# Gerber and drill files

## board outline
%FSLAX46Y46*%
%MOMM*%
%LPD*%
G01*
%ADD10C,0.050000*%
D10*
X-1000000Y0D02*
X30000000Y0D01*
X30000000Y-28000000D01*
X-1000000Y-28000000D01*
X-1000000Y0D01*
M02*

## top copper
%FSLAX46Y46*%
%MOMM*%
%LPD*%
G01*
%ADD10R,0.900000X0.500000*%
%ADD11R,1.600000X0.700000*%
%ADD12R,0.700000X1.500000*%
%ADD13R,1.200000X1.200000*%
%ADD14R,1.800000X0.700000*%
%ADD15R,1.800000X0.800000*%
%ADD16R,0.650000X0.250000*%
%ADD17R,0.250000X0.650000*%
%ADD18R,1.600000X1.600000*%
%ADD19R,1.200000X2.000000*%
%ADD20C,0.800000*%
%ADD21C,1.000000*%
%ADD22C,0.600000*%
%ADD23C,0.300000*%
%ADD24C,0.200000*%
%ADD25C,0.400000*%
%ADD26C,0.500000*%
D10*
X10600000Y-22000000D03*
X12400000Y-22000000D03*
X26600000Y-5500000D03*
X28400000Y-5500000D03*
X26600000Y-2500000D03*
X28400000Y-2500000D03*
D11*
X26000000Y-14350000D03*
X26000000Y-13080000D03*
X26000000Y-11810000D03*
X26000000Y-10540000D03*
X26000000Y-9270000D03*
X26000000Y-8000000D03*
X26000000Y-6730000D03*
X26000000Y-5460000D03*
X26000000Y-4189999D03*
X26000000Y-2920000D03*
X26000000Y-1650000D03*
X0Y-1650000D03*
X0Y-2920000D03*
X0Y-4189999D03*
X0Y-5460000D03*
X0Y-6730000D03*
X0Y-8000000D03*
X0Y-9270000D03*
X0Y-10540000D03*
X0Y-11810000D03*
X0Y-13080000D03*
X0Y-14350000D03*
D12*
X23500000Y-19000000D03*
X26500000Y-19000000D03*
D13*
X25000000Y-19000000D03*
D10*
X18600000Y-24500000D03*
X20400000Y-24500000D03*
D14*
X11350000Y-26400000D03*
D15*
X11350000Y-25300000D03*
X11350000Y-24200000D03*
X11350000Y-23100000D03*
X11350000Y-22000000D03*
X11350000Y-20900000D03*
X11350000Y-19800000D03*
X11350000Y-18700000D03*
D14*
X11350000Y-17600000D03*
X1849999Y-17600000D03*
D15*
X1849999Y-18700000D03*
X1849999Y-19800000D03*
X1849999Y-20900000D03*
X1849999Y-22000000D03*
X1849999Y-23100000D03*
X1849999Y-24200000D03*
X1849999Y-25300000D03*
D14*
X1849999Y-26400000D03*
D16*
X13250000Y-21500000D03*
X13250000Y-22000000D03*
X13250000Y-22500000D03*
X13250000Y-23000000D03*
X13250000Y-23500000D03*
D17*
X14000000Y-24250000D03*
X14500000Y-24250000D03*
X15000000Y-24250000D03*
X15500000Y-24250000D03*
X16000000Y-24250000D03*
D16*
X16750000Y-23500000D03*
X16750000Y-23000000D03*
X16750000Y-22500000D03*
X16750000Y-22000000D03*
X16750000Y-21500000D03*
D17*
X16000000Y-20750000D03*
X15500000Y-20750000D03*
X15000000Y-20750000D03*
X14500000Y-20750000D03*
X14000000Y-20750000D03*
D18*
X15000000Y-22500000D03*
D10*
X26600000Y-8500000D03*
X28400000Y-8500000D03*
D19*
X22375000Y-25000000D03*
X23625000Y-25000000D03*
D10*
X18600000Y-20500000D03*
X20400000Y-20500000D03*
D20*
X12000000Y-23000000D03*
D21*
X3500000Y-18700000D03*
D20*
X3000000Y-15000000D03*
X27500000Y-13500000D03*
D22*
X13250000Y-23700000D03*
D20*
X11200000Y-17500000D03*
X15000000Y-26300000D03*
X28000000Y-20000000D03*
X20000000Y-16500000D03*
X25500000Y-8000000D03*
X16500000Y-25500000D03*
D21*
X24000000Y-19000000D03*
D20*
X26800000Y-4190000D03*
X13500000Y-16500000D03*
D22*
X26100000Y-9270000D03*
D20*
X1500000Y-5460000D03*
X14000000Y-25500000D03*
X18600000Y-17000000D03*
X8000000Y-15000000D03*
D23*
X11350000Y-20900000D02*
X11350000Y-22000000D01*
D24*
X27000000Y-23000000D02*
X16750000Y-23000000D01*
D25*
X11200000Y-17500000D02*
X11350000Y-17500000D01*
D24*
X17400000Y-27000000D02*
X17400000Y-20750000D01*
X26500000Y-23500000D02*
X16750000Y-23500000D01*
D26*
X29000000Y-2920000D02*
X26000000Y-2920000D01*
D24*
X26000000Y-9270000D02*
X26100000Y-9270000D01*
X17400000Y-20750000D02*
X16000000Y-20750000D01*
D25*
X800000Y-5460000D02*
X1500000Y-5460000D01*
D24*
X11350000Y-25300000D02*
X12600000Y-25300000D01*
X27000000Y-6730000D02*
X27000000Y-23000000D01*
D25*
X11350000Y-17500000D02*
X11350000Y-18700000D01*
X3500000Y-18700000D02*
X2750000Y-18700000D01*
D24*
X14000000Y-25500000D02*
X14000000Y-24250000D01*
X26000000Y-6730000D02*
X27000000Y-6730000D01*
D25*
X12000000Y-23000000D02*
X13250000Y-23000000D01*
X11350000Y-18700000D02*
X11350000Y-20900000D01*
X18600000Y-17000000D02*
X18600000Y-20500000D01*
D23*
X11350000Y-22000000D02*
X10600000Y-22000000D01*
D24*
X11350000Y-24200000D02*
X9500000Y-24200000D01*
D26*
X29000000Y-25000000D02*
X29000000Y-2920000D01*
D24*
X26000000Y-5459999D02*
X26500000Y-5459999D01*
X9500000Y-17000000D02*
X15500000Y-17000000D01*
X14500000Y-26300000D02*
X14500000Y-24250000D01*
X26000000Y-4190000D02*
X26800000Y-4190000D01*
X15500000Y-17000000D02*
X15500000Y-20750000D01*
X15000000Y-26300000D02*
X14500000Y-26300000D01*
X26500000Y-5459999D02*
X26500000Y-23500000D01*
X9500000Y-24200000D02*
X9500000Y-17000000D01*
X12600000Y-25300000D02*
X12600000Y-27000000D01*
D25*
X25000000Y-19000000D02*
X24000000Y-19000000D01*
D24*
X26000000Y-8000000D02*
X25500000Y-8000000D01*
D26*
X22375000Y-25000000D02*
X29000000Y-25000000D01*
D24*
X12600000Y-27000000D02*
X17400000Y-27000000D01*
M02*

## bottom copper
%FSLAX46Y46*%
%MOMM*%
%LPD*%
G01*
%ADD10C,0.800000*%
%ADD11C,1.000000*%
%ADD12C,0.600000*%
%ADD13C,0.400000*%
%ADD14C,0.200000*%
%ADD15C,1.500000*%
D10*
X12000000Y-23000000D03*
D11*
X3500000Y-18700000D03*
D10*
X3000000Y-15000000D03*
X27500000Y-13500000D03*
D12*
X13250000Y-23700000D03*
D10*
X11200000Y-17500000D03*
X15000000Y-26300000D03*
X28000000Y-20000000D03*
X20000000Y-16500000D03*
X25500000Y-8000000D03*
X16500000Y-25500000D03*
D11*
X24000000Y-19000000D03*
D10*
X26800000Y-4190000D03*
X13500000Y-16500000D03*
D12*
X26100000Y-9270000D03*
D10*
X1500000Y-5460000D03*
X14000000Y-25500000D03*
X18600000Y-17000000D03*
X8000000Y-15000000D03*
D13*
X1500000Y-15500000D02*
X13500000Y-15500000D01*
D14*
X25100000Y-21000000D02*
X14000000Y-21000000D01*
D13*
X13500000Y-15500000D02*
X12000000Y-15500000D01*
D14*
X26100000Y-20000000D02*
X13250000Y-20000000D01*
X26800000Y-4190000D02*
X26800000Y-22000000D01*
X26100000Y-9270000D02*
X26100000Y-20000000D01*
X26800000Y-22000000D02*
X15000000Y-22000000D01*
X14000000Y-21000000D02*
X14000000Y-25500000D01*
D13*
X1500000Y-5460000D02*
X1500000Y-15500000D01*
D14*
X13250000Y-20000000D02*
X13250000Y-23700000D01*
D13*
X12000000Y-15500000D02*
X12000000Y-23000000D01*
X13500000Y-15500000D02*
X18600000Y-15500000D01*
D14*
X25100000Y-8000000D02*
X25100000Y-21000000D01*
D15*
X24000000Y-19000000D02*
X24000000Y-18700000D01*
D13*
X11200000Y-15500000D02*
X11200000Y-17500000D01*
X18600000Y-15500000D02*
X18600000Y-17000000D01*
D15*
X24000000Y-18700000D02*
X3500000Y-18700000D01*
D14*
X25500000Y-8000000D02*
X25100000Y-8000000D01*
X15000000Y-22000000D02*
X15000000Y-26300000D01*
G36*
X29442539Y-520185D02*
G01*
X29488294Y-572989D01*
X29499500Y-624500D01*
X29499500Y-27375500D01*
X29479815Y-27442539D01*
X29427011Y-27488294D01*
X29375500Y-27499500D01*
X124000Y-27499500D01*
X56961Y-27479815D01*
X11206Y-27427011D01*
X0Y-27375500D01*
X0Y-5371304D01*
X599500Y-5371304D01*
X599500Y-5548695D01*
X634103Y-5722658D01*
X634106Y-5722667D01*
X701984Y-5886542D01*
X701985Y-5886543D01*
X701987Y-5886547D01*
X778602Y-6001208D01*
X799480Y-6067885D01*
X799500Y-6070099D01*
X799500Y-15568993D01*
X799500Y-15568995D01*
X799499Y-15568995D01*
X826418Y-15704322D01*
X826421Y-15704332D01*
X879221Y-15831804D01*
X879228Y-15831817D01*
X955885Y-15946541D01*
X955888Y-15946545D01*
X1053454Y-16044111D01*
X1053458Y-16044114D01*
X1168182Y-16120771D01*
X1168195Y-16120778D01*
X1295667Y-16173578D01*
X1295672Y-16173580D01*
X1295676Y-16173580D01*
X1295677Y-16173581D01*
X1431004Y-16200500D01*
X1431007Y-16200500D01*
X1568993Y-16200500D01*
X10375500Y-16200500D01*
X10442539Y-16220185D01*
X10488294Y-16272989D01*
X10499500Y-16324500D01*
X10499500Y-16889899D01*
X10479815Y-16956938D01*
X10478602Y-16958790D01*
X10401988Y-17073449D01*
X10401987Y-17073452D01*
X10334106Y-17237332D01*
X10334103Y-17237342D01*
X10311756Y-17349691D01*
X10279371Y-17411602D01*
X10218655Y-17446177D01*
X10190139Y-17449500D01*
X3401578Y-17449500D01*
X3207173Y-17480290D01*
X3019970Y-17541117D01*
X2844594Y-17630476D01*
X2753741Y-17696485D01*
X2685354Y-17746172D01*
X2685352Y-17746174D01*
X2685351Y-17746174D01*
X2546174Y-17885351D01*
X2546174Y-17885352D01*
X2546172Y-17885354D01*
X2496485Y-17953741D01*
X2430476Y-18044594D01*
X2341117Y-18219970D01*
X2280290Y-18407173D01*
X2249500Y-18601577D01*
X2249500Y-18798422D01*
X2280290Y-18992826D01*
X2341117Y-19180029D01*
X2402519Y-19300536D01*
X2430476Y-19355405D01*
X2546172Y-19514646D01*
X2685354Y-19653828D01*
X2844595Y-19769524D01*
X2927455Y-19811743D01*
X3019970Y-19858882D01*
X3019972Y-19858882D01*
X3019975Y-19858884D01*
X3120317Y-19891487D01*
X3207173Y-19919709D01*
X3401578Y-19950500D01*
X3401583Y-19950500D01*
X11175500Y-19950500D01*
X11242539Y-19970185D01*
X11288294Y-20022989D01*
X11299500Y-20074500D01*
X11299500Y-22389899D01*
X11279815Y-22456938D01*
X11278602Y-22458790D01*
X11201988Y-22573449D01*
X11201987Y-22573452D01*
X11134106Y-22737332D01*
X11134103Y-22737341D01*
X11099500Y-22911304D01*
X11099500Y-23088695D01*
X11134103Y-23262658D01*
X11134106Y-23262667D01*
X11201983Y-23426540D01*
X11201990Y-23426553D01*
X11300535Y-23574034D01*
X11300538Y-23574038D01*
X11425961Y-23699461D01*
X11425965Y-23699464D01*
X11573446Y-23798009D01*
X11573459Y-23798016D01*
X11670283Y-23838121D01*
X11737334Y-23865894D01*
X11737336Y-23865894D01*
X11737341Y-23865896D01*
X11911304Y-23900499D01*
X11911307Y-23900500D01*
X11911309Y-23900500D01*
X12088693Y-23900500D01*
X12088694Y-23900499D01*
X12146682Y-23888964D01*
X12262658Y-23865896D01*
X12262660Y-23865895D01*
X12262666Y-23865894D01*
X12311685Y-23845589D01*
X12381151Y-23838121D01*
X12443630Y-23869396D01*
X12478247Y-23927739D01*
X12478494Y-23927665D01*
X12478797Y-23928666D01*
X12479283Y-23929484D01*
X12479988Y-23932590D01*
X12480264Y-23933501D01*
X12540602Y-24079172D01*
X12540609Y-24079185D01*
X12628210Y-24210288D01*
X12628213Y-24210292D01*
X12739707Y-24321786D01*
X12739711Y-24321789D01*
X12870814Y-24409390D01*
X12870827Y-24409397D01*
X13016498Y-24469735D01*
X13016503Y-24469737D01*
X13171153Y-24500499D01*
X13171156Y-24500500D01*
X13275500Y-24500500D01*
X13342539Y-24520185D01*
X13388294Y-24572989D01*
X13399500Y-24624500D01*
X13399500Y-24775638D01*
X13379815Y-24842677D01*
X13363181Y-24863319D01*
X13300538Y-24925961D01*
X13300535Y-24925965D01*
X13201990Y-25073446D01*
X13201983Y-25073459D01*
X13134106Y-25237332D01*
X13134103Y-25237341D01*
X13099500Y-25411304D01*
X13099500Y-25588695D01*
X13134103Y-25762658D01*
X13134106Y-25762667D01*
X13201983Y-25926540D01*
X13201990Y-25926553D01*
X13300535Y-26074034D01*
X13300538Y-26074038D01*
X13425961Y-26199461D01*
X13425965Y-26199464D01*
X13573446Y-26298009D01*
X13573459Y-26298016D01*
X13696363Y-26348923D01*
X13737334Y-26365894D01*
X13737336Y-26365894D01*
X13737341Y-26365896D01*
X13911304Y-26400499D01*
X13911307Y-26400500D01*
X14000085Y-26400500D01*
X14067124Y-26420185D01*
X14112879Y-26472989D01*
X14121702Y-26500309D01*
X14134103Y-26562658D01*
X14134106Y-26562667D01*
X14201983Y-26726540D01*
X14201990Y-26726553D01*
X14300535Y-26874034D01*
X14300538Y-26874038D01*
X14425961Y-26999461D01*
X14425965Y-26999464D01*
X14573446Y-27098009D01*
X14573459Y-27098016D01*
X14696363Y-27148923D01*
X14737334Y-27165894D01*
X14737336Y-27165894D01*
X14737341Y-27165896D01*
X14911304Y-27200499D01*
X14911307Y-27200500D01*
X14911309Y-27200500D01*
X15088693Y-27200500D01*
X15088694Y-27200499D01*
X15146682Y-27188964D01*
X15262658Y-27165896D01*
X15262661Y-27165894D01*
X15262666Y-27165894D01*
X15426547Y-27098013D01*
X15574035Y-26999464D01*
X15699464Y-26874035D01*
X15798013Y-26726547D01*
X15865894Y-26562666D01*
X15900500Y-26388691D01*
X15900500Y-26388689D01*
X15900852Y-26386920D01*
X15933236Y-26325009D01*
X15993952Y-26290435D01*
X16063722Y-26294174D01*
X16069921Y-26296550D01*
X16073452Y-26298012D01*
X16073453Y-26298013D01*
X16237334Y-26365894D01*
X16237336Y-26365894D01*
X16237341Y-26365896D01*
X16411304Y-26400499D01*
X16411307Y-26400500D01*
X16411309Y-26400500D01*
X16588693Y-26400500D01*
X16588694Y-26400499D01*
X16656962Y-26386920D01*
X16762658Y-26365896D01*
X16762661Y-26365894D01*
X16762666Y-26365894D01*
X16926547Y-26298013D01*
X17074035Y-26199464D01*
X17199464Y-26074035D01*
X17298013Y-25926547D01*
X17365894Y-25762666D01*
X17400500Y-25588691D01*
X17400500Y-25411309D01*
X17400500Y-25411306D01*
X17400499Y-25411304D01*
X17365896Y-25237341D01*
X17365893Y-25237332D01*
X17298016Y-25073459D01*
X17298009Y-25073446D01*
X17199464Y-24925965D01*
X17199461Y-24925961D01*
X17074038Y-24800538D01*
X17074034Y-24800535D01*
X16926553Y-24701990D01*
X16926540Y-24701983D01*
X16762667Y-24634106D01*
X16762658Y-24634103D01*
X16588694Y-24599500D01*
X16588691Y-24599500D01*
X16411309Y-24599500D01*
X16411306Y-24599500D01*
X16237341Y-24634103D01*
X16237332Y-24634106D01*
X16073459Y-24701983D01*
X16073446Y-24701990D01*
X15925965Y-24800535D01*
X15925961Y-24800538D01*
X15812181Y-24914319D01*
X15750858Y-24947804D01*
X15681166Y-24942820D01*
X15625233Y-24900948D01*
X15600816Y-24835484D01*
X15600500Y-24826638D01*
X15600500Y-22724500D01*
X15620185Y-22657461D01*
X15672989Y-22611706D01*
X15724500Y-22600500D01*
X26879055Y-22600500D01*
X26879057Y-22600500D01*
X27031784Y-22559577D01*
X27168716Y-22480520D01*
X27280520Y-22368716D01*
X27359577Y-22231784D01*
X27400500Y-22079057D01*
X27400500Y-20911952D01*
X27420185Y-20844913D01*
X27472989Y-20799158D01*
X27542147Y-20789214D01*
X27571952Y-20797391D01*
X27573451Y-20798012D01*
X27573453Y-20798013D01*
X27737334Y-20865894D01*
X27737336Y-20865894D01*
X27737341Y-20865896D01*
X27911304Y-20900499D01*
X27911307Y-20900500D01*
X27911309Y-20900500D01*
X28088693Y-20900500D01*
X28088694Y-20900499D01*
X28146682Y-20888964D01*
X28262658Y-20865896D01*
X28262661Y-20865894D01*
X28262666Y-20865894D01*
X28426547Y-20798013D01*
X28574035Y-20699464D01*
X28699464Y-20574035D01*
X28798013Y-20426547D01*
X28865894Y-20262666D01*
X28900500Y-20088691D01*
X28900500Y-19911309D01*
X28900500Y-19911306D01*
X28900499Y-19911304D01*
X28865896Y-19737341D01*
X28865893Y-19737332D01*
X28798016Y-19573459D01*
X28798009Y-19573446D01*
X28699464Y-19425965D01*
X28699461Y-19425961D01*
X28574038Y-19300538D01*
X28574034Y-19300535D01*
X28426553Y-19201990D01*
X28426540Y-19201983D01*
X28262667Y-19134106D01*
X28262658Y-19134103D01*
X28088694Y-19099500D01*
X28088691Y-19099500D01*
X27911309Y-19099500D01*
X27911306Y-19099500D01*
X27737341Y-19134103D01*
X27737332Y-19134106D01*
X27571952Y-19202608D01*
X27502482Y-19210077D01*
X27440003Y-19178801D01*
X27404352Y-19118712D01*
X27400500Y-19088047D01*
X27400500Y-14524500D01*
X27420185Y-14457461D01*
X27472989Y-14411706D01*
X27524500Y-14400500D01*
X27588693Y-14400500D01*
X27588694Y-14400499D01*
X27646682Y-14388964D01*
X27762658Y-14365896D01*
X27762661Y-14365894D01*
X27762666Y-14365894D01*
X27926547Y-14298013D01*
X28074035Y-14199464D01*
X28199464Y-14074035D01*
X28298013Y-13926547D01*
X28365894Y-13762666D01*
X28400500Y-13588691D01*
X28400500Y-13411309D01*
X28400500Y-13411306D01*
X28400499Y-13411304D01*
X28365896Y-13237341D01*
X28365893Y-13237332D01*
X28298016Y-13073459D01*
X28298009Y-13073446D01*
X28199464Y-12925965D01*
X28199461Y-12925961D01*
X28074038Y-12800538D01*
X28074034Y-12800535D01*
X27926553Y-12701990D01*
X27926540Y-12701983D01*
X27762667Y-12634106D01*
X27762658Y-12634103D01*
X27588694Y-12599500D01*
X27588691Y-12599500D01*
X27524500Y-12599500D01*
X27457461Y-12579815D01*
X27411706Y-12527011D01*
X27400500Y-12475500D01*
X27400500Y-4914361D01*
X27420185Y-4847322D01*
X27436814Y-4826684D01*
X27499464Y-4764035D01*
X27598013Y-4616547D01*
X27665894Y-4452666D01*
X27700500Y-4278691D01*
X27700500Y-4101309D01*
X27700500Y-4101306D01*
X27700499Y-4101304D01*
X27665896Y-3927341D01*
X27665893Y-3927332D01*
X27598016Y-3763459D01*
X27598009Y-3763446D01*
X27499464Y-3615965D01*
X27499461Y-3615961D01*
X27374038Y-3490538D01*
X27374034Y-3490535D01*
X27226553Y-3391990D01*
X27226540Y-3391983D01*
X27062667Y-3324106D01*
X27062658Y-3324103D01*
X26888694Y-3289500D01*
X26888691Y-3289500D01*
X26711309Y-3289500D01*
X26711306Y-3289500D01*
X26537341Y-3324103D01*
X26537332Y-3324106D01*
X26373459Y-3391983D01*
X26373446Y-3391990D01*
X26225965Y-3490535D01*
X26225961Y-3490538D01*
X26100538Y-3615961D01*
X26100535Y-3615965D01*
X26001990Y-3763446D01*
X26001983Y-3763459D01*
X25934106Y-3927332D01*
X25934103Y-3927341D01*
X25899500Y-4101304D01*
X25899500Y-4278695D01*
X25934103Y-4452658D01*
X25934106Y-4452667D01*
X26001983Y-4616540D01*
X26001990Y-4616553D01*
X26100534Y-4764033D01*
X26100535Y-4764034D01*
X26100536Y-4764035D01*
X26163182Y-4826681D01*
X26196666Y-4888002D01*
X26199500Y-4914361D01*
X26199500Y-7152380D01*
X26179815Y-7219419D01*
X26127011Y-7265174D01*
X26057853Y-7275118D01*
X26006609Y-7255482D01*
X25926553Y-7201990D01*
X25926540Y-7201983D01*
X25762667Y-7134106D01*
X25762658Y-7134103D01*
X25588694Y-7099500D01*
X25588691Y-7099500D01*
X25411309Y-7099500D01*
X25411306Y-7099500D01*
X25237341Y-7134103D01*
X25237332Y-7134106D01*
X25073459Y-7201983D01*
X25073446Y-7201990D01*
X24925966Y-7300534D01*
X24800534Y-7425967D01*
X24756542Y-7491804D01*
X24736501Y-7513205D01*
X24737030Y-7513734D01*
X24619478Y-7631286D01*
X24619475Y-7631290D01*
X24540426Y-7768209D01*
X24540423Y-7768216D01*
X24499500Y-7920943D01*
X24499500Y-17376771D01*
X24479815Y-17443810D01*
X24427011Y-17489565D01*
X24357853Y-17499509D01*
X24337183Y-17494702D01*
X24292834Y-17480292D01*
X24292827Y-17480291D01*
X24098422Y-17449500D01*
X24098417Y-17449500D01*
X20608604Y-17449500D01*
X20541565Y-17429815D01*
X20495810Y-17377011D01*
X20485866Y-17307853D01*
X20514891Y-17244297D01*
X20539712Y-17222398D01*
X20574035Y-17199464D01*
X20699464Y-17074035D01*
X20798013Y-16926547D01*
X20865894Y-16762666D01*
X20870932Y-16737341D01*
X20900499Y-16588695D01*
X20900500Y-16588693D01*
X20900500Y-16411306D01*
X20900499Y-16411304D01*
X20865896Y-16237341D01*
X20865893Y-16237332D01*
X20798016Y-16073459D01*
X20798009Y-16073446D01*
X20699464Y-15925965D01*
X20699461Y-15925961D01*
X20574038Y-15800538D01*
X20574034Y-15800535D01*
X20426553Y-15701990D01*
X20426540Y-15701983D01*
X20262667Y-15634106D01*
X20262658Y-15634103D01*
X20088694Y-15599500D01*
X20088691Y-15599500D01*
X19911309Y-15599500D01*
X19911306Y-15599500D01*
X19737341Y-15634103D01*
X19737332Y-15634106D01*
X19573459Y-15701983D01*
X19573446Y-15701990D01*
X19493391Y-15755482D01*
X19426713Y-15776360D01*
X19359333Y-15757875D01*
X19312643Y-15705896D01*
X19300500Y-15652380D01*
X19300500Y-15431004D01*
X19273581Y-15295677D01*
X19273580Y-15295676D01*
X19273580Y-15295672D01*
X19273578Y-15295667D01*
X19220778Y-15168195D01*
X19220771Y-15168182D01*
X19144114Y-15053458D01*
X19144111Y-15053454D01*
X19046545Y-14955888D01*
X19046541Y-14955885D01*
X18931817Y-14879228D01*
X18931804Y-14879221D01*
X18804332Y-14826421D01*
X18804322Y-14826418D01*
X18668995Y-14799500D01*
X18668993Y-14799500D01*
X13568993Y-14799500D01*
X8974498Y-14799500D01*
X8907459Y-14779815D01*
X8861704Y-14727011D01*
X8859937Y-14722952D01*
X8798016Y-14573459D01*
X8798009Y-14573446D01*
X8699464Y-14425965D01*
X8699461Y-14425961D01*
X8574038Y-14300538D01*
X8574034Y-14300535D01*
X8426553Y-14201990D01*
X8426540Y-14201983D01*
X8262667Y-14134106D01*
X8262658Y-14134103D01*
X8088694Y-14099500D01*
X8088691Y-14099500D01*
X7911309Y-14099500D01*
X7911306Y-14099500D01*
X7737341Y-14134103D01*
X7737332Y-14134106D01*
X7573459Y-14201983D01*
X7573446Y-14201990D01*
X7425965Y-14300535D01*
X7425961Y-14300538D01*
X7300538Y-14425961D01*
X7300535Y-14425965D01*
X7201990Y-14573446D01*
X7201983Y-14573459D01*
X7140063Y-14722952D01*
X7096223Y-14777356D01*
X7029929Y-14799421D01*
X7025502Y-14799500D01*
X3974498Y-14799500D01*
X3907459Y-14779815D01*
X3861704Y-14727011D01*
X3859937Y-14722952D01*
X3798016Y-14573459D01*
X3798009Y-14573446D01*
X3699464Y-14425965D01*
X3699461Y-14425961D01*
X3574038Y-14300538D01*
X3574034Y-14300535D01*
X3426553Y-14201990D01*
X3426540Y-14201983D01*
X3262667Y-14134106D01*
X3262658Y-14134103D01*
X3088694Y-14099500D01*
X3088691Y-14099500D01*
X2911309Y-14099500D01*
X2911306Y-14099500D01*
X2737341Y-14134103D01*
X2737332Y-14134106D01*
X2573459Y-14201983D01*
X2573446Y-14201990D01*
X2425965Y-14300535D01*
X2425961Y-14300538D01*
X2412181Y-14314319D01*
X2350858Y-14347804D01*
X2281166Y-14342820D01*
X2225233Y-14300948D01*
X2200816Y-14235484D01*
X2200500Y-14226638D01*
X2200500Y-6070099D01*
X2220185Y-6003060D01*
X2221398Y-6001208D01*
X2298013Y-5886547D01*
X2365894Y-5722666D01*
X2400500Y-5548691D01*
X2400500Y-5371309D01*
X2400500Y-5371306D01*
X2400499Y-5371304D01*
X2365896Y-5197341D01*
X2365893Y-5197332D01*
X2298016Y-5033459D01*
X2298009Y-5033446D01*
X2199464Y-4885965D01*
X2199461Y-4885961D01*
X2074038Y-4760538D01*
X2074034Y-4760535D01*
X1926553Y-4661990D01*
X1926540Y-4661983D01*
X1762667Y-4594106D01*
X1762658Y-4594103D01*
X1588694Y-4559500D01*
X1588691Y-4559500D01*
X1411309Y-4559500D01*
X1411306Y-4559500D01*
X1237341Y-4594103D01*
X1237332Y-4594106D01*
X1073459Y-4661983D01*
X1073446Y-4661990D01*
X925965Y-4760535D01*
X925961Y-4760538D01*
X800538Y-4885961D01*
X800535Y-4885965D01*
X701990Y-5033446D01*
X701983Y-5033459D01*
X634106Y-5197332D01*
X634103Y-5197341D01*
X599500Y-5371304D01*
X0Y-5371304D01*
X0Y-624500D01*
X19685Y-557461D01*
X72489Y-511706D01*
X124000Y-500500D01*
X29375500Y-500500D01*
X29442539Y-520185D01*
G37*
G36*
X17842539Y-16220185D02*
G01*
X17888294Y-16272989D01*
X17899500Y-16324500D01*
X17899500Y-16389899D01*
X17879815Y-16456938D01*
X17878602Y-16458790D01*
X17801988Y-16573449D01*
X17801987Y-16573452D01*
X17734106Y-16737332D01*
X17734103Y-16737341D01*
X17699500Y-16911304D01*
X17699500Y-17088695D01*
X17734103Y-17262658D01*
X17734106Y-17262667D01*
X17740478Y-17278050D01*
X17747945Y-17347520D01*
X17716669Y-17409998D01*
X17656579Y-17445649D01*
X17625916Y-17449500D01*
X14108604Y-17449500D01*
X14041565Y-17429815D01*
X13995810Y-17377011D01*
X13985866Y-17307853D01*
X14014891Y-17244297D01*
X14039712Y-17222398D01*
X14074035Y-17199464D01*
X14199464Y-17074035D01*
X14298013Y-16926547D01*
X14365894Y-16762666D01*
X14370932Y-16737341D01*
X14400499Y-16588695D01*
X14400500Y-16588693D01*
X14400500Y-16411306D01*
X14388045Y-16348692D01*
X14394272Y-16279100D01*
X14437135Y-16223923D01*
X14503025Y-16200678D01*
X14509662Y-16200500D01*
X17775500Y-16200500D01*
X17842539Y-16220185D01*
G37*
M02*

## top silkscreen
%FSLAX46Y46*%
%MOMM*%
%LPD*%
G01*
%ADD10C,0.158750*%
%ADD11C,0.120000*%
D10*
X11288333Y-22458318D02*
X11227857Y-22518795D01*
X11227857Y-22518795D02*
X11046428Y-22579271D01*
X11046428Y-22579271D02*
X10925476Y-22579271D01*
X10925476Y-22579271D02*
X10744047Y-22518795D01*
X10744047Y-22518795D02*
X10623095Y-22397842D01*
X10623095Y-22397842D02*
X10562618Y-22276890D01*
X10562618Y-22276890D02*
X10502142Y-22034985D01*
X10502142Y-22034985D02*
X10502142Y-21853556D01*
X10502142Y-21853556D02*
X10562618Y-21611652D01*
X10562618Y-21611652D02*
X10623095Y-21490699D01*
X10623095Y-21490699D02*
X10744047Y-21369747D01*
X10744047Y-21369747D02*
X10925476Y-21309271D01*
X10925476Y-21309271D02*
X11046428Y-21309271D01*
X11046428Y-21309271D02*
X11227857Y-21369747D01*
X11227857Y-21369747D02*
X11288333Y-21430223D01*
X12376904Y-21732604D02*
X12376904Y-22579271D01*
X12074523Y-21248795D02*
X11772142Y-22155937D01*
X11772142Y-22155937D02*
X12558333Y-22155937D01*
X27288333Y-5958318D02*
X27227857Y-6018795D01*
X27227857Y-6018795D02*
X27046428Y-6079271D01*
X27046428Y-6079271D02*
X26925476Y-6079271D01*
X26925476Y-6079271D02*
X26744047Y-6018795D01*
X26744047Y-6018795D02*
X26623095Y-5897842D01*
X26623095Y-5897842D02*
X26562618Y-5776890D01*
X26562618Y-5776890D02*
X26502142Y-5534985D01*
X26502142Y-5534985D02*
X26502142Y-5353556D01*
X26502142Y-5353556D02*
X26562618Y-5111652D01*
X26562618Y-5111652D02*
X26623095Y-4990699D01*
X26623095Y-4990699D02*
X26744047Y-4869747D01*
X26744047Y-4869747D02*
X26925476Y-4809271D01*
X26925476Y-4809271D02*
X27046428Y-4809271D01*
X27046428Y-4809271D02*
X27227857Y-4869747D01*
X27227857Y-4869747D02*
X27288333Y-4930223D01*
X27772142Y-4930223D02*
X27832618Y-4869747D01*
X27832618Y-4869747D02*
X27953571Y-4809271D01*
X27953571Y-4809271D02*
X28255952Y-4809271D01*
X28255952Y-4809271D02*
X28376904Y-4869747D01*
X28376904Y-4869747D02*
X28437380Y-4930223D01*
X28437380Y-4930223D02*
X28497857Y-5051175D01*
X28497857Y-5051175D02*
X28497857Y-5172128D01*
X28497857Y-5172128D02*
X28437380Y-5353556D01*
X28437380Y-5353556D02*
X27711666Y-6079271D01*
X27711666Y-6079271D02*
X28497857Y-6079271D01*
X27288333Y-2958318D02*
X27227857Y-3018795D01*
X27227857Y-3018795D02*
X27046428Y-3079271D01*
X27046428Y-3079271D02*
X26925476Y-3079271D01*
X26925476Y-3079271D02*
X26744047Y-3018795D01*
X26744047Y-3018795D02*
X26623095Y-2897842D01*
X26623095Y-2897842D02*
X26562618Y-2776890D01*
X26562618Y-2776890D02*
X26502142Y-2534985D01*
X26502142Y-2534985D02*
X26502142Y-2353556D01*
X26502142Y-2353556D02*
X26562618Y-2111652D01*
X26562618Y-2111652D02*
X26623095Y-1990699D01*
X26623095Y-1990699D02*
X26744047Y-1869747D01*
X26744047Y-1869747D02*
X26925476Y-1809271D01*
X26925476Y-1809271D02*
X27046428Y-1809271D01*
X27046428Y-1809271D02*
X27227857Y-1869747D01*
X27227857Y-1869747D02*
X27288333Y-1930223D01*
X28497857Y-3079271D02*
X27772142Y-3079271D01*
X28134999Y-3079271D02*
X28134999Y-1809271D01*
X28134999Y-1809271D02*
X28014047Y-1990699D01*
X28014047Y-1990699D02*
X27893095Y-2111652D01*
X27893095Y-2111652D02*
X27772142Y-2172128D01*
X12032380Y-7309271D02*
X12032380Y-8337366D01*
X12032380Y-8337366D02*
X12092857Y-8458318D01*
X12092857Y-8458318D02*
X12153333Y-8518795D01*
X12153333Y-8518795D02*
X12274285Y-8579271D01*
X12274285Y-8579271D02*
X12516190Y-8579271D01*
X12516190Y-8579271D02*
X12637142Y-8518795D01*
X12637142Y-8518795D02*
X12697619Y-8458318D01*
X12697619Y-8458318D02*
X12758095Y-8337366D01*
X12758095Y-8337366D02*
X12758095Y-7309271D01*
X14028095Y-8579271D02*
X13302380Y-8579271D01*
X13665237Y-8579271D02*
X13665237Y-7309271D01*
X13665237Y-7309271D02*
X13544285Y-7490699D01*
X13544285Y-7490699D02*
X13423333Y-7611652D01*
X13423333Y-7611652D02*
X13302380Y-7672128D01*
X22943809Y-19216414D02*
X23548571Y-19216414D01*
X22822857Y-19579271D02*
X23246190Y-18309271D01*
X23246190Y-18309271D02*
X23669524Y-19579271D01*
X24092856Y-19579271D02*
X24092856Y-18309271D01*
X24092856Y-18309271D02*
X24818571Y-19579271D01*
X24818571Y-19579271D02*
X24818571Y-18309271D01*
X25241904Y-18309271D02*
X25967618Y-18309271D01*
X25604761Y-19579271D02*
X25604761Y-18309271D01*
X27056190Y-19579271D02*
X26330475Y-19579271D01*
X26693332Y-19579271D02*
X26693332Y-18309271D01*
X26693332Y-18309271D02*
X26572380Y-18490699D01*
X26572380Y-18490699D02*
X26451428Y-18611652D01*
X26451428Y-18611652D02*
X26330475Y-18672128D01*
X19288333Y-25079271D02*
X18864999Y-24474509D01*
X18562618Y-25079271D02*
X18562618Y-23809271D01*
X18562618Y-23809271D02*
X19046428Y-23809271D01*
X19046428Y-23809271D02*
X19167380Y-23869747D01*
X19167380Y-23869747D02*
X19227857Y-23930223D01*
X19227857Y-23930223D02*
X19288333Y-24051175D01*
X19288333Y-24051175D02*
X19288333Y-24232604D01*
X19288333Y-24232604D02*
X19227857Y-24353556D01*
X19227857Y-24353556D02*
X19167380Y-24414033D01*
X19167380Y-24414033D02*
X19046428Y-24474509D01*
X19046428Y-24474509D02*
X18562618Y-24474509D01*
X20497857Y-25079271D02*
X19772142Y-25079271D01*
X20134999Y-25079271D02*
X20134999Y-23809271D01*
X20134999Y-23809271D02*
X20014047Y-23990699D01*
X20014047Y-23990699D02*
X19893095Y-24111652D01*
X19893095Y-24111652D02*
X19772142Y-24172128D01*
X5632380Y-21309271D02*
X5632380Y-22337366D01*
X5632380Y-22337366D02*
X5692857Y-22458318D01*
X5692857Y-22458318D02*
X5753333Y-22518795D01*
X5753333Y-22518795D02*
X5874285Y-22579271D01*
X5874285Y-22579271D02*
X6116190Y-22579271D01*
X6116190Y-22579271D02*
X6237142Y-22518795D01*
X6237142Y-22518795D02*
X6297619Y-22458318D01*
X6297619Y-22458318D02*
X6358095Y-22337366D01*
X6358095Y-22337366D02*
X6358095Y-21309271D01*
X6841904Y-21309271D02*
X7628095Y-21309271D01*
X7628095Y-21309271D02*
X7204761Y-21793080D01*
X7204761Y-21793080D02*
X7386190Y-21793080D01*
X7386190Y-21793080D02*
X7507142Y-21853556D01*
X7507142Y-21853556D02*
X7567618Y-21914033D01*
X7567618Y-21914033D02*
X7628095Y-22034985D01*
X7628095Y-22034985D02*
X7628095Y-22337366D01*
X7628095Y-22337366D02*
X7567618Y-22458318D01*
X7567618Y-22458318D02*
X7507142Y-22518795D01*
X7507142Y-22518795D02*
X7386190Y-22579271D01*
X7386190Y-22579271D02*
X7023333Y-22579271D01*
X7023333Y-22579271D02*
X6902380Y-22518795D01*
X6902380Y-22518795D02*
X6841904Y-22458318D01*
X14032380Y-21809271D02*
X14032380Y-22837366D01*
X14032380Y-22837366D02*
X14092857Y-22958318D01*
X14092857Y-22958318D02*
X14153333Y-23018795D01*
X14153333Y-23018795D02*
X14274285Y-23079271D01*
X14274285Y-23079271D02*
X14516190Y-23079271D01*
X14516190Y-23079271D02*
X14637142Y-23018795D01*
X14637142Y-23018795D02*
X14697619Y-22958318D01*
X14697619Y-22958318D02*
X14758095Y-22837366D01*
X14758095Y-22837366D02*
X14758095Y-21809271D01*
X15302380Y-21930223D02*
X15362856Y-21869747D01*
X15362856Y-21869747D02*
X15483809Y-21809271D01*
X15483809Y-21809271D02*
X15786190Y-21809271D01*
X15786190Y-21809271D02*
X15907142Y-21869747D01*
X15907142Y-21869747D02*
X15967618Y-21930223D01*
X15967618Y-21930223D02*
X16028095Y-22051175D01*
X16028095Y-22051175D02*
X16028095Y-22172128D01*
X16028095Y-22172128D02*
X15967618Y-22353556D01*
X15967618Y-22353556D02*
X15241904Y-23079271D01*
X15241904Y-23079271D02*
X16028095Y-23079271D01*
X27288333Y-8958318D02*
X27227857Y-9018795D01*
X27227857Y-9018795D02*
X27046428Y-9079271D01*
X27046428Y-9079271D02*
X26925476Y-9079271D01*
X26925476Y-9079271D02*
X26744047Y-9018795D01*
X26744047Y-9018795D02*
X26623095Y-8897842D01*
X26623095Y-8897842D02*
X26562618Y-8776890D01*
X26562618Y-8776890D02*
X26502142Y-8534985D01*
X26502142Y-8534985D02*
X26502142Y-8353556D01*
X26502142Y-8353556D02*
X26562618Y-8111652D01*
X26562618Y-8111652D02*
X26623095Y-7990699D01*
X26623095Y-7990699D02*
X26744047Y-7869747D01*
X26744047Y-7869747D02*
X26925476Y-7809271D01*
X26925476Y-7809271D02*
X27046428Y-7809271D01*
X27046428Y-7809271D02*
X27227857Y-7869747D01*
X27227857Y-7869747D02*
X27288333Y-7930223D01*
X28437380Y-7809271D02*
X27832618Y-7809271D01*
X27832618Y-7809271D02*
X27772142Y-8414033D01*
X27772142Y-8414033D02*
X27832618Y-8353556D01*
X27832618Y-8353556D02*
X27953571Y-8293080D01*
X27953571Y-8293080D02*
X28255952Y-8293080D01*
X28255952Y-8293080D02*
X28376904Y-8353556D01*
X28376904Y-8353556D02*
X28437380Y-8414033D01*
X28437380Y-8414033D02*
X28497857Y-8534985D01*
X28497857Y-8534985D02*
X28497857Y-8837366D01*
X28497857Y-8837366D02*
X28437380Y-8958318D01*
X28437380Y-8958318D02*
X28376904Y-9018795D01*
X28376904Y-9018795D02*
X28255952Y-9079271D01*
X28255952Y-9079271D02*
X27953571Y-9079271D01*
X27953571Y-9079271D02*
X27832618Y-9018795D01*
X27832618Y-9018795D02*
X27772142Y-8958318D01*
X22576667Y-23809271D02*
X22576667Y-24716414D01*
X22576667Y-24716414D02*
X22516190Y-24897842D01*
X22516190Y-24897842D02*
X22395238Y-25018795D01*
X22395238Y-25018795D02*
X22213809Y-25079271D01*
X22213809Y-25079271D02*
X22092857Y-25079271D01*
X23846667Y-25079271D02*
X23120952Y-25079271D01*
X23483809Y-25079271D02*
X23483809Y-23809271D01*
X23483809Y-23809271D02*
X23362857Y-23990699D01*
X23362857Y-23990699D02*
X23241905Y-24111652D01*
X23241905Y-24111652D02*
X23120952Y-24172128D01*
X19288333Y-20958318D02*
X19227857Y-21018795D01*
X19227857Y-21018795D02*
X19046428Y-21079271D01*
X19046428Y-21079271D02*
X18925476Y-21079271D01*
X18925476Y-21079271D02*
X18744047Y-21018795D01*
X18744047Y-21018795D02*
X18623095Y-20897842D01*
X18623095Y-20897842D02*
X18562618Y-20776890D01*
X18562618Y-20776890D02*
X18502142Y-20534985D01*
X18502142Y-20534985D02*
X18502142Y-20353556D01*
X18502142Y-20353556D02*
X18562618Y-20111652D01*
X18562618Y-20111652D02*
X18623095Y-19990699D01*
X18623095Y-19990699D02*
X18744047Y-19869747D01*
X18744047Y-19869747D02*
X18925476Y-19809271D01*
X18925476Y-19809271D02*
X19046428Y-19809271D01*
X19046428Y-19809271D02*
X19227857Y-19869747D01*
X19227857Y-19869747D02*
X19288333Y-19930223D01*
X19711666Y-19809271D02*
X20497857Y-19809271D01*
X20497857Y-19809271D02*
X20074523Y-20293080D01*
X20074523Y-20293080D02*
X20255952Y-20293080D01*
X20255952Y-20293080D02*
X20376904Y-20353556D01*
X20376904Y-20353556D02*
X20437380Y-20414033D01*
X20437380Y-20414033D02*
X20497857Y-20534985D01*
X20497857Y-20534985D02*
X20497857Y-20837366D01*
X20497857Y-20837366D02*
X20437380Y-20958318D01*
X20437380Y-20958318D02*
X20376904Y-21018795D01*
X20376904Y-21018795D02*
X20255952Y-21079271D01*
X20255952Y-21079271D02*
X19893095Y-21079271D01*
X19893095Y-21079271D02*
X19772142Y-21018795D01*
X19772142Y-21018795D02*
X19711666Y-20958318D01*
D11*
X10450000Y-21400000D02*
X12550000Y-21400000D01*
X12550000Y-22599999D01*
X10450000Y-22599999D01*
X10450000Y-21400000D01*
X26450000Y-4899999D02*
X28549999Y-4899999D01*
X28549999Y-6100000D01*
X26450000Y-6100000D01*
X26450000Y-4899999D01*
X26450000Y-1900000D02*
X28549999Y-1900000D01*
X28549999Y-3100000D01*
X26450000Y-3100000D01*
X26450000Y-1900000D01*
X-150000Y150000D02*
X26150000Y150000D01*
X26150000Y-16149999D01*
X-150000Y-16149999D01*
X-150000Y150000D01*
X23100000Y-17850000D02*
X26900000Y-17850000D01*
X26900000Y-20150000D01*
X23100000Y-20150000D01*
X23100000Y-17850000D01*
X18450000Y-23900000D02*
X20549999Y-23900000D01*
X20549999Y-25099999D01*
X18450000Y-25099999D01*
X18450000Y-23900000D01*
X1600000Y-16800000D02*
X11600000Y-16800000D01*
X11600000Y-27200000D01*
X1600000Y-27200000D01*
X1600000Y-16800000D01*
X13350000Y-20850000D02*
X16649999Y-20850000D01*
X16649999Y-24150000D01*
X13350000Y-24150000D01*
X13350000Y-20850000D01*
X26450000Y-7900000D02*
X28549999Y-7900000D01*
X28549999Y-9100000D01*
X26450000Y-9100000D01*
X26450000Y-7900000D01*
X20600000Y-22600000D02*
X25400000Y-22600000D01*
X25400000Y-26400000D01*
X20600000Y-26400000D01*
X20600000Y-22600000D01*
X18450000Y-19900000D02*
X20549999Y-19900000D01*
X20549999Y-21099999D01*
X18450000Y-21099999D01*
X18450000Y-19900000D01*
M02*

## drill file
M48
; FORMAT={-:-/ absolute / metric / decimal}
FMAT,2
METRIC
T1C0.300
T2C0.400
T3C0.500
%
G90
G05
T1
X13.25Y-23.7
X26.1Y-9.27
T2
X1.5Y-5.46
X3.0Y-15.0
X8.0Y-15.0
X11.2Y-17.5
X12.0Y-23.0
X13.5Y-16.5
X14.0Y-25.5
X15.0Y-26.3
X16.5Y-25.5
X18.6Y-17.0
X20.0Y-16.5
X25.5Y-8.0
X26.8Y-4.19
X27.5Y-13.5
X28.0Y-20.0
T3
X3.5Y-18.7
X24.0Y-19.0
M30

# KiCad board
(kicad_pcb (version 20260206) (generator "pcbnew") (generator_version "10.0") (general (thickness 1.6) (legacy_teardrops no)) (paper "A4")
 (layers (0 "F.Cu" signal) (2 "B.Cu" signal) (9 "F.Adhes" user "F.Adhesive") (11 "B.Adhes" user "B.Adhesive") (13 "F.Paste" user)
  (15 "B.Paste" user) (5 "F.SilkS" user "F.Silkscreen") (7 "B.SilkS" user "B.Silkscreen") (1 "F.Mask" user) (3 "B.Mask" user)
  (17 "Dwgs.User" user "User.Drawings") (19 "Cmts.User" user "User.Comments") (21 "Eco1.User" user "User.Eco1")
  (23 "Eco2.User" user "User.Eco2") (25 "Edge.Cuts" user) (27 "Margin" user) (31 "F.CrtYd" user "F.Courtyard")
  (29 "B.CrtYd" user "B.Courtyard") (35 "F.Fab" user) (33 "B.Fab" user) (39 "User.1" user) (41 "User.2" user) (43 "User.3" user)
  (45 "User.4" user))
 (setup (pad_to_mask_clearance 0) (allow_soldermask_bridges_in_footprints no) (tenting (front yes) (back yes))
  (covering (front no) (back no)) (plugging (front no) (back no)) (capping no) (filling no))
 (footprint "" (layer "F.Cu") (at 11.5 22)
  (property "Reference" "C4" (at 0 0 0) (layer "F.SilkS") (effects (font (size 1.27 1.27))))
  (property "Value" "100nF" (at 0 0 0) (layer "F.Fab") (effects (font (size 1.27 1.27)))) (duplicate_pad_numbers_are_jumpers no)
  (fp_rect (start -1.05 -0.6) (end 1.05 0.599999) (stroke (width 0.12) (type default)) (fill no) (layer "F.SilkS"))
  (pad "1" smd rect (at -0.9 0) (size 0.9 0.5) (layers "F.Cu" "F.Mask" "F.Paste") (thermal_bridge_angle 45))
  (pad "2" smd rect (at 0.9 0) (size 0.9 0.5) (layers "F.Cu" "F.Mask" "F.Paste") (thermal_bridge_angle 45)))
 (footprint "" (layer "F.Cu") (at 27.5 5.5)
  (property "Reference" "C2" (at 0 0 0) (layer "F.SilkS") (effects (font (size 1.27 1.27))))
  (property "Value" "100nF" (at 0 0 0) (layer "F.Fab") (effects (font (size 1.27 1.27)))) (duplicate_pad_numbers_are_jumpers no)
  (fp_rect (start -1.05 -0.600001) (end 1.049999 0.6) (stroke (width 0.12) (type default)) (fill no) (layer "F.SilkS"))
  (pad "1" smd rect (at -0.9 0) (size 0.9 0.5) (layers "F.Cu" "F.Mask" "F.Paste") (thermal_bridge_angle 45))
  (pad "2" smd rect (at 0.9 0) (size 0.9 0.5) (layers "F.Cu" "F.Mask" "F.Paste") (thermal_bridge_angle 45)))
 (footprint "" (layer "F.Cu") (at 27.5 2.5)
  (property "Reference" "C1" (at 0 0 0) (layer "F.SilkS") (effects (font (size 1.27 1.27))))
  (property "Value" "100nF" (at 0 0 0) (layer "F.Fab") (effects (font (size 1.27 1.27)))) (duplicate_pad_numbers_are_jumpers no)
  (fp_rect (start -1.05 -0.6) (end 1.049999 0.6) (stroke (width 0.12) (type default)) (fill no) (layer "F.SilkS"))
  (pad "1" smd rect (at -0.9 0) (size 0.9 0.5) (layers "F.Cu" "F.Mask" "F.Paste") (thermal_bridge_angle 45))
  (pad "2" smd rect (at 0.9 0) (size 0.9 0.5) (layers "F.Cu" "F.Mask" "F.Paste") (thermal_bridge_angle 45)))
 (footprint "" (layer "F.Cu") (at 13 8)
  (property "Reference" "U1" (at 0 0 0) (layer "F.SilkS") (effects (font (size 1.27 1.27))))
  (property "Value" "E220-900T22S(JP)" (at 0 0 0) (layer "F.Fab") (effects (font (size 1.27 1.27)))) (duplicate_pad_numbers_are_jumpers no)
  (fp_rect (start -13.15 -8.15) (end 13.15 8.149999) (stroke (width 0.12) (type default)) (fill no) (layer "F.SilkS"))
  (pad "1" smd rect (at 13 6.35) (size 1.6 0.7) (layers "F.Cu" "F.Mask" "F.Paste") (thermal_bridge_angle 45))
  (pad "2" smd rect (at 13 5.08) (size 1.6 0.7) (layers "F.Cu" "F.Mask" "F.Paste") (thermal_bridge_angle 45))
  (pad "3" smd rect (at 13 3.81) (size 1.6 0.7) (layers "F.Cu" "F.Mask" "F.Paste") (thermal_bridge_angle 45))
  (pad "4" smd rect (at 13 2.54) (size 1.6 0.7) (layers "F.Cu" "F.Mask" "F.Paste") (thermal_bridge_angle 45))
  (pad "5" smd rect (at 13 1.27) (size 1.6 0.7) (layers "F.Cu" "F.Mask" "F.Paste") (thermal_bridge_angle 45))
  (pad "6" smd rect (at 13 0) (size 1.6 0.7) (layers "F.Cu" "F.Mask" "F.Paste") (thermal_bridge_angle 45))
  (pad "7" smd rect (at 13 -1.27) (size 1.6 0.7) (layers "F.Cu" "F.Mask" "F.Paste") (thermal_bridge_angle 45))
  (pad "8" smd rect (at 13 -2.54) (size 1.6 0.7) (layers "F.Cu" "F.Mask" "F.Paste") (thermal_bridge_angle 45))
  (pad "9" smd rect (at 13 -3.810001) (size 1.6 0.7) (layers "F.Cu" "F.Mask" "F.Paste") (thermal_bridge_angle 45))
  (pad "10" smd rect (at 13 -5.08) (size 1.6 0.7) (layers "F.Cu" "F.Mask" "F.Paste") (thermal_bridge_angle 45))
  (pad "11" smd rect (at 13 -6.35) (size 1.6 0.7) (layers "F.Cu" "F.Mask" "F.Paste") (thermal_bridge_angle 45))
  (pad "12" smd rect (at -13 -6.35) (size 1.6 0.7) (layers "F.Cu" "F.Mask" "F.Paste") (thermal_bridge_angle 45))
  (pad "13" smd rect (at -13 -5.08) (size 1.6 0.7) (layers "F.Cu" "F.Mask" "F.Paste") (thermal_bridge_angle 45))
  (pad "14" smd rect (at -13 -3.810001) (size 1.6 0.7) (layers "F.Cu" "F.Mask" "F.Paste") (thermal_bridge_angle 45))
  (pad "15" smd rect (at -13 -2.54) (size 1.6 0.7) (layers "F.Cu" "F.Mask" "F.Paste") (thermal_bridge_angle 45))
  (pad "16" smd rect (at -13 -1.27) (size 1.6 0.7) (layers "F.Cu" "F.Mask" "F.Paste") (thermal_bridge_angle 45))
  (pad "17" smd rect (at -13 0) (size 1.6 0.7) (layers "F.Cu" "F.Mask" "F.Paste") (thermal_bridge_angle 45))
  (pad "18" smd rect (at -13 1.27) (size 1.6 0.7) (layers "F.Cu" "F.Mask" "F.Paste") (thermal_bridge_angle 45))
  (pad "19" smd rect (at -13 2.54) (size 1.6 0.7) (layers "F.Cu" "F.Mask" "F.Paste") (thermal_bridge_angle 45))
  (pad "20" smd rect (at -13 3.81) (size 1.6 0.7) (layers "F.Cu" "F.Mask" "F.Paste") (thermal_bridge_angle 45))
  (pad "21" smd rect (at -13 5.08) (size 1.6 0.7) (layers "F.Cu" "F.Mask" "F.Paste") (thermal_bridge_angle 45))
  (pad "22" smd rect (at -13 6.35) (size 1.6 0.7) (layers "F.Cu" "F.Mask" "F.Paste") (thermal_bridge_angle 45)))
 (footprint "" (layer "F.Cu") (at 25 19)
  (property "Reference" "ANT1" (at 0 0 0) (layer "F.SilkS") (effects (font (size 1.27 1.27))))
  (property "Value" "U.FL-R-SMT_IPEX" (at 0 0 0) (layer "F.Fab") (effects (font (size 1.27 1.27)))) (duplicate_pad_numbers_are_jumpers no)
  (fp_rect (start -1.9 -1.15) (end 1.9 1.15) (stroke (width 0.12) (type default)) (fill no) (layer "F.SilkS"))
  (pad "G1" smd rect (at -1.5 0) (size 0.7 1.5) (layers "F.Cu" "F.Mask" "F.Paste") (thermal_bridge_angle 45))
  (pad "G2" smd rect (at 1.5 0) (size 0.7 1.5) (layers "F.Cu" "F.Mask" "F.Paste") (thermal_bridge_angle 45))
  (pad "S" smd rect (at 0 0) (size 1.2 1.2) (layers "F.Cu" "F.Mask" "F.Paste") (thermal_bridge_angle 45)))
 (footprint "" (layer "F.Cu") (at 19.5 24.5)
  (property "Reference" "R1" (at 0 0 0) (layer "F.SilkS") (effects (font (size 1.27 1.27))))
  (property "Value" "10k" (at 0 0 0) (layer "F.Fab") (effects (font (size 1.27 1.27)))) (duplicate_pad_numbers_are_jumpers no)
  (fp_rect (start -1.05 -0.6) (end 1.049999 0.599999) (stroke (width 0.12) (type default)) (fill no) (layer "F.SilkS"))
  (pad "1" smd rect (at -0.9 0) (size 0.9 0.5) (layers "F.Cu" "F.Mask" "F.Paste") (thermal_bridge_angle 45))
  (pad "2" smd rect (at 0.9 0) (size 0.9 0.5) (layers "F.Cu" "F.Mask" "F.Paste") (thermal_bridge_angle 45)))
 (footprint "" (layer "F.Cu") (at 6.6 22)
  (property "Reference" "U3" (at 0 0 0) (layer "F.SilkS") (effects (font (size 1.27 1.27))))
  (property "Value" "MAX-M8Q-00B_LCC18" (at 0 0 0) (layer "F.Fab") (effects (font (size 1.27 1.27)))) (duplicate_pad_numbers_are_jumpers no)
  (fp_rect (start -5 -5.2) (end 5 5.2) (stroke (width 0.12) (type default)) (fill no) (layer "F.SilkS"))
  (pad "1" smd rect (at 4.75 4.4) (size 1.8 0.7) (layers "F.Cu" "F.Mask" "F.Paste") (thermal_bridge_angle 45))
  (pad "2" smd rect (at 4.75 3.3) (size 1.8 0.8) (layers "F.Cu" "F.Mask" "F.Paste") (thermal_bridge_angle 45))
  (pad "3" smd rect (at 4.75 2.2) (size 1.8 0.8) (layers "F.Cu" "F.Mask" "F.Paste") (thermal_bridge_angle 45))
  (pad "4" smd rect (at 4.75 1.1) (size 1.8 0.8) (layers "F.Cu" "F.Mask" "F.Paste") (thermal_bridge_angle 45))
  (pad "5" smd rect (at 4.75 0) (size 1.8 0.8) (layers "F.Cu" "F.Mask" "F.Paste") (thermal_bridge_angle 45))
  (pad "6" smd rect (at 4.75 -1.1) (size 1.8 0.8) (layers "F.Cu" "F.Mask" "F.Paste") (thermal_bridge_angle 45))
  (pad "7" smd rect (at 4.75 -2.2) (size 1.8 0.8) (layers "F.Cu" "F.Mask" "F.Paste") (thermal_bridge_angle 45))
  (pad "8" smd rect (at 4.75 -3.3) (size 1.8 0.8) (layers "F.Cu" "F.Mask" "F.Paste") (thermal_bridge_angle 45))
  (pad "9" smd rect (at 4.75 -4.4) (size 1.8 0.7) (layers "F.Cu" "F.Mask" "F.Paste") (thermal_bridge_angle 45))
  (pad "10" smd rect (at -4.750001 -4.4) (size 1.8 0.7) (layers "F.Cu" "F.Mask" "F.Paste") (thermal_bridge_angle 45))
  (pad "11" smd rect (at -4.750001 -3.3) (size 1.8 0.8) (layers "F.Cu" "F.Mask" "F.Paste") (thermal_bridge_angle 45))
  (pad "12" smd rect (at -4.750001 -2.2) (size 1.8 0.8) (layers "F.Cu" "F.Mask" "F.Paste") (thermal_bridge_angle 45))
  (pad "13" smd rect (at -4.750001 -1.1) (size 1.8 0.8) (layers "F.Cu" "F.Mask" "F.Paste") (thermal_bridge_angle 45))
  (pad "14" smd rect (at -4.750001 0) (size 1.8 0.8) (layers "F.Cu" "F.Mask" "F.Paste") (thermal_bridge_angle 45))
  (pad "15" smd rect (at -4.750001 1.1) (size 1.8 0.8) (layers "F.Cu" "F.Mask" "F.Paste") (thermal_bridge_angle 45))
  (pad "16" smd rect (at -4.750001 2.2) (size 1.8 0.8) (layers "F.Cu" "F.Mask" "F.Paste") (thermal_bridge_angle 45))
  (pad "17" smd rect (at -4.750001 3.3) (size 1.8 0.8) (layers "F.Cu" "F.Mask" "F.Paste") (thermal_bridge_angle 45))
  (pad "18" smd rect (at -4.750001 4.4) (size 1.8 0.7) (layers "F.Cu" "F.Mask" "F.Paste") (thermal_bridge_angle 45)))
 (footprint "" (layer "F.Cu") (at 15 22.5)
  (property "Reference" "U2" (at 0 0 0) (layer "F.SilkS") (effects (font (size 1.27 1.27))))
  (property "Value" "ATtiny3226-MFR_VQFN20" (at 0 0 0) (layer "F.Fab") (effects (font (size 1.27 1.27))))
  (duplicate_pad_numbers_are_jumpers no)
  (fp_rect (start -1.65 -1.65) (end 1.649999 1.65) (stroke (width 0.12) (type default)) (fill no) (layer "F.SilkS"))
  (pad "1" smd rect (at -1.75 -1) (size 0.65 0.25) (layers "F.Cu" "F.Mask" "F.Paste") (thermal_bridge_angle 45))
  (pad "2" smd rect (at -1.75 -0.5) (size 0.65 0.25) (layers "F.Cu" "F.Mask" "F.Paste") (thermal_bridge_angle 45))
  (pad "3" smd rect (at -1.75 0) (size 0.65 0.25) (layers "F.Cu" "F.Mask" "F.Paste") (thermal_bridge_angle 45))
  (pad "4" smd rect (at -1.75 0.5) (size 0.65 0.25) (layers "F.Cu" "F.Mask" "F.Paste") (thermal_bridge_angle 45))
  (pad "5" smd rect (at -1.75 1) (size 0.65 0.25) (layers "F.Cu" "F.Mask" "F.Paste") (thermal_bridge_angle 45))
  (pad "6" smd rect (at -1 1.75) (size 0.25 0.65) (layers "F.Cu" "F.Mask" "F.Paste") (thermal_bridge_angle 45))
  (pad "7" smd rect (at -0.5 1.75) (size 0.25 0.65) (layers "F.Cu" "F.Mask" "F.Paste") (thermal_bridge_angle 45))
  (pad "8" smd rect (at 0 1.75) (size 0.25 0.65) (layers "F.Cu" "F.Mask" "F.Paste") (thermal_bridge_angle 45))
  (pad "9" smd rect (at 0.5 1.75) (size 0.25 0.65) (layers "F.Cu" "F.Mask" "F.Paste") (thermal_bridge_angle 45))
  (pad "10" smd rect (at 1 1.75) (size 0.25 0.65) (layers "F.Cu" "F.Mask" "F.Paste") (thermal_bridge_angle 45))
  (pad "11" smd rect (at 1.75 1) (size 0.65 0.25) (layers "F.Cu" "F.Mask" "F.Paste") (thermal_bridge_angle 45))
  (pad "12" smd rect (at 1.75 0.5) (size 0.65 0.25) (layers "F.Cu" "F.Mask" "F.Paste") (thermal_bridge_angle 45))
  (pad "13" smd rect (at 1.75 0) (size 0.65 0.25) (layers "F.Cu" "F.Mask" "F.Paste") (thermal_bridge_angle 45))
  (pad "14" smd rect (at 1.75 -0.5) (size 0.65 0.25) (layers "F.Cu" "F.Mask" "F.Paste") (thermal_bridge_angle 45))
  (pad "15" smd rect (at 1.75 -1) (size 0.65 0.25) (layers "F.Cu" "F.Mask" "F.Paste") (thermal_bridge_angle 45))
  (pad "16" smd rect (at 1 -1.75) (size 0.25 0.65) (layers "F.Cu" "F.Mask" "F.Paste") (thermal_bridge_angle 45))
  (pad "17" smd rect (at 0.5 -1.75) (size 0.25 0.65) (layers "F.Cu" "F.Mask" "F.Paste") (thermal_bridge_angle 45))
  (pad "18" smd rect (at 0 -1.75) (size 0.25 0.65) (layers "F.Cu" "F.Mask" "F.Paste") (thermal_bridge_angle 45))
  (pad "19" smd rect (at -0.5 -1.75) (size 0.25 0.65) (layers "F.Cu" "F.Mask" "F.Paste") (thermal_bridge_angle 45))
  (pad "20" smd rect (at -1 -1.75) (size 0.25 0.65) (layers "F.Cu" "F.Mask" "F.Paste") (thermal_bridge_angle 45))
  (pad "EP" smd rect (at 0 0) (size 1.6 1.6) (layers "F.Cu" "F.Mask" "F.Paste") (thermal_bridge_angle 45)))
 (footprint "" (layer "F.Cu") (at 27.5 8.5)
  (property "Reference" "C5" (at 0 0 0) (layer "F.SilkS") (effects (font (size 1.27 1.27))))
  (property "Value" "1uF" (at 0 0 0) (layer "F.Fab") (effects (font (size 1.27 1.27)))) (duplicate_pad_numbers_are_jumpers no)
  (fp_rect (start -1.05 -0.6) (end 1.049999 0.6) (stroke (width 0.12) (type default)) (fill no) (layer "F.SilkS"))
  (pad "1" smd rect (at -0.9 0) (size 0.9 0.5) (layers "F.Cu" "F.Mask" "F.Paste") (thermal_bridge_angle 45))
  (pad "2" smd rect (at 0.9 0) (size 0.9 0.5) (layers "F.Cu" "F.Mask" "F.Paste") (thermal_bridge_angle 45)))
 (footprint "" (layer "F.Cu") (at 23 24.5)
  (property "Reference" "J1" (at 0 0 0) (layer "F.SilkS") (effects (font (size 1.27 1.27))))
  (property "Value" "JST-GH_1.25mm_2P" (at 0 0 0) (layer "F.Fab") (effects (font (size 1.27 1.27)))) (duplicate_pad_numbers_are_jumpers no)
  (fp_rect (start -2.4 -1.9) (end 2.4 1.9) (stroke (width 0.12) (type default)) (fill no) (layer "F.SilkS"))
  (pad "1" smd rect (at -0.625 0.5) (size 1.2 2) (layers "F.Cu" "F.Mask" "F.Paste") (thermal_bridge_angle 45))
  (pad "2" smd rect (at 0.625 0.5) (size 1.2 2) (layers "F.Cu" "F.Mask" "F.Paste") (thermal_bridge_angle 45)))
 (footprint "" (layer "F.Cu") (at 19.5 20.5)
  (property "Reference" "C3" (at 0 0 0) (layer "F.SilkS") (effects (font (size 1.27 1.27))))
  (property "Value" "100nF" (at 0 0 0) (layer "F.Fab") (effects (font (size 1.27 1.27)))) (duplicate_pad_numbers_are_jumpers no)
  (fp_rect (start -1.05 -0.6) (end 1.049999 0.599999) (stroke (width 0.12) (type default)) (fill no) (layer "F.SilkS"))
  (pad "1" smd rect (at -0.9 0) (size 0.9 0.5) (layers "F.Cu" "F.Mask" "F.Paste") (thermal_bridge_angle 45))
  (pad "2" smd rect (at 0.9 0) (size 0.9 0.5) (layers "F.Cu" "F.Mask" "F.Paste") (thermal_bridge_angle 45)))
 (gr_rect (start -1 0) (end 30 28) (stroke (width 0.05) (type default)) (fill no) (layer "Edge.Cuts"))
 (segment (start 11.35 20.9) (end 11.35 22) (width 0.3) (layer "F.Cu") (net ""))
 (segment (start 27 23) (end 16.75 23) (width 0.2) (layer "F.Cu") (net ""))
 (segment (start 11.2 17.5) (end 11.35 17.5) (width 0.4) (layer "F.Cu") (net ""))
 (segment (start 17.4 27) (end 17.4 20.75) (width 0.2) (layer "F.Cu") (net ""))
 (segment (start 26.5 23.5) (end 16.75 23.5) (width 0.2) (layer "F.Cu") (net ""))
 (segment (start 29 2.92) (end 26 2.92) (width 0.5) (layer "F.Cu") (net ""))
 (segment (start 26 9.27) (end 26.1 9.27) (width 0.2) (layer "F.Cu") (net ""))
 (segment (start 17.4 20.75) (end 16 20.75) (width 0.2) (layer "F.Cu") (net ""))
 (segment (start 0.8 5.46) (end 1.5 5.46) (width 0.4) (layer "F.Cu") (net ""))
 (segment (start 11.35 25.3) (end 12.6 25.3) (width 0.2) (layer "F.Cu") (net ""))
 (segment (start 27 6.73) (end 27 23) (width 0.2) (layer "F.Cu") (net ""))
 (segment (start 11.35 17.5) (end 11.35 18.7) (width 0.4) (layer "F.Cu") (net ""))
 (segment (start 3.5 18.7) (end 2.75 18.7) (width 0.4) (layer "F.Cu") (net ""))
 (segment (start 14 25.5) (end 14 24.25) (width 0.2) (layer "F.Cu") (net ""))
 (segment (start 26 6.73) (end 27 6.73) (width 0.2) (layer "F.Cu") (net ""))
 (segment (start 12 23) (end 13.25 23) (width 0.4) (layer "F.Cu") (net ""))
 (segment (start 11.35 18.7) (end 11.35 20.9) (width 0.4) (layer "F.Cu") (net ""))
 (segment (start 18.6 17) (end 18.6 20.5) (width 0.4) (layer "F.Cu") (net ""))
 (segment (start 11.35 22) (end 10.6 22) (width 0.3) (layer "F.Cu") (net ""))
 (segment (start 11.35 24.2) (end 9.5 24.2) (width 0.2) (layer "F.Cu") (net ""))
 (segment (start 29 25) (end 29 2.92) (width 0.5) (layer "F.Cu") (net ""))
 (segment (start 26 5.459999) (end 26.5 5.459999) (width 0.2) (layer "F.Cu") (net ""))
 (segment (start 9.5 17) (end 15.5 17) (width 0.2) (layer "F.Cu") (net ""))
 (segment (start 14.5 26.3) (end 14.5 24.25) (width 0.2) (layer "F.Cu") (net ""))
 (segment (start 26 4.19) (end 26.8 4.19) (width 0.2) (layer "F.Cu") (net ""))
 (segment (start 15.5 17) (end 15.5 20.75) (width 0.2) (layer "F.Cu") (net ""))
 (segment (start 15 26.3) (end 14.5 26.3) (width 0.2) (layer "F.Cu") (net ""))
 (segment (start 26.5 5.459999) (end 26.5 23.5) (width 0.2) (layer "F.Cu") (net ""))
 (segment (start 9.5 24.2) (end 9.5 17) (width 0.2) (layer "F.Cu") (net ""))
 (segment (start 12.6 25.3) (end 12.6 27) (width 0.2) (layer "F.Cu") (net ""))
 (segment (start 25 19) (end 24 19) (width 0.4) (layer "F.Cu") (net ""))
 (segment (start 26 8) (end 25.5 8) (width 0.2) (layer "F.Cu") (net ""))
 (segment (start 22.375 25) (end 29 25) (width 0.5) (layer "F.Cu") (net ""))
 (segment (start 12.6 27) (end 17.4 27) (width 0.2) (layer "F.Cu") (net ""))
 (via (at 12 23) (size 0.8) (drill 0.4) (layers "F.Cu" "B.Cu") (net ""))
 (via (at 3.5 18.7) (size 1) (drill 0.5) (layers "F.Cu" "B.Cu") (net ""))
 (via (at 3 15) (size 0.8) (drill 0.4) (layers "F.Cu" "B.Cu") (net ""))
 (via (at 27.5 13.5) (size 0.8) (drill 0.4) (layers "F.Cu" "B.Cu") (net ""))
 (via (at 13.25 23.7) (size 0.6) (drill 0.3) (layers "F.Cu" "B.Cu") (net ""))
 (via (at 11.2 17.5) (size 0.8) (drill 0.4) (layers "F.Cu" "B.Cu") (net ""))
 (via (at 15 26.3) (size 0.8) (drill 0.4) (layers "F.Cu" "B.Cu") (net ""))
 (via (at 28 20) (size 0.8) (drill 0.4) (layers "F.Cu" "B.Cu") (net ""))
 (via (at 20 16.5) (size 0.8) (drill 0.4) (layers "F.Cu" "B.Cu") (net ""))
 (via (at 25.5 8) (size 0.8) (drill 0.4) (layers "F.Cu" "B.Cu") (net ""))
 (via (at 16.5 25.5) (size 0.8) (drill 0.4) (layers "F.Cu" "B.Cu") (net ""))
 (via (at 24 19) (size 1) (drill 0.5) (layers "F.Cu" "B.Cu") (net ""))
 (via (at 26.8 4.19) (size 0.8) (drill 0.4) (layers "F.Cu" "B.Cu") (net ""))
 (via (at 13.5 16.5) (size 0.8) (drill 0.4) (layers "F.Cu" "B.Cu") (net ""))
 (via (at 26.1 9.27) (size 0.6) (drill 0.3) (layers "F.Cu" "B.Cu") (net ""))
 (via (at 1.5 5.46) (size 0.8) (drill 0.4) (layers "F.Cu" "B.Cu") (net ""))
 (via (at 14 25.5) (size 0.8) (drill 0.4) (layers "F.Cu" "B.Cu") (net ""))
 (via (at 18.6 17) (size 0.8) (drill 0.4) (layers "F.Cu" "B.Cu") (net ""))
 (via (at 8 15) (size 0.8) (drill 0.4) (layers "F.Cu" "B.Cu") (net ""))
 (segment (start 1.5 15.5) (end 13.5 15.5) (width 0.4) (layer "B.Cu") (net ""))
 (segment (start 25.1 21) (end 14 21) (width 0.2) (layer "B.Cu") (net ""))
 (segment (start 13.5 15.5) (end 12 15.5) (width 0.4) (layer "B.Cu") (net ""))
 (segment (start 26.1 20) (end 13.25 20) (width 0.2) (layer "B.Cu") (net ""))
 (segment (start 26.8 4.19) (end 26.8 22) (width 0.2) (layer "B.Cu") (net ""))
 (segment (start 26.1 9.27) (end 26.1 20) (width 0.2) (layer "B.Cu") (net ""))
 (segment (start 26.8 22) (end 15 22) (width 0.2) (layer "B.Cu") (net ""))
 (segment (start 14 21) (end 14 25.5) (width 0.2) (layer "B.Cu") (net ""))
 (segment (start 1.5 5.46) (end 1.5 15.5) (width 0.4) (layer "B.Cu") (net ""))
 (segment (start 13.25 20) (end 13.25 23.7) (width 0.2) (layer "B.Cu") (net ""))
 (segment (start 12 15.5) (end 12 23) (width 0.4) (layer "B.Cu") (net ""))
 (segment (start 13.5 15.5) (end 18.6 15.5) (width 0.4) (layer "B.Cu") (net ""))
 (segment (start 25.1 8) (end 25.1 21) (width 0.2) (layer "B.Cu") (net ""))
 (segment (start 24 19) (end 24 18.7) (width 1.5) (layer "B.Cu") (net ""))
 (segment (start 11.2 15.5) (end 11.2 17.5) (width 0.4) (layer "B.Cu") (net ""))
 (segment (start 18.6 15.5) (end 18.6 17) (width 0.4) (layer "B.Cu") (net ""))
 (segment (start 24 18.7) (end 3.5 18.7) (width 1.5) (layer "B.Cu") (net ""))
 (segment (start 25.5 8) (end 25.1 8) (width 0.2) (layer "B.Cu") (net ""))
 (segment (start 15 22) (end 15 26.3) (width 0.2) (layer "B.Cu") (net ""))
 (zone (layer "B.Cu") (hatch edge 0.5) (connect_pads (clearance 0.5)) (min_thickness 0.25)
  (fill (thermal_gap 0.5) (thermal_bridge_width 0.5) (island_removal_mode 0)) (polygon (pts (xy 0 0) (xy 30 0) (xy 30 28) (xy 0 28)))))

